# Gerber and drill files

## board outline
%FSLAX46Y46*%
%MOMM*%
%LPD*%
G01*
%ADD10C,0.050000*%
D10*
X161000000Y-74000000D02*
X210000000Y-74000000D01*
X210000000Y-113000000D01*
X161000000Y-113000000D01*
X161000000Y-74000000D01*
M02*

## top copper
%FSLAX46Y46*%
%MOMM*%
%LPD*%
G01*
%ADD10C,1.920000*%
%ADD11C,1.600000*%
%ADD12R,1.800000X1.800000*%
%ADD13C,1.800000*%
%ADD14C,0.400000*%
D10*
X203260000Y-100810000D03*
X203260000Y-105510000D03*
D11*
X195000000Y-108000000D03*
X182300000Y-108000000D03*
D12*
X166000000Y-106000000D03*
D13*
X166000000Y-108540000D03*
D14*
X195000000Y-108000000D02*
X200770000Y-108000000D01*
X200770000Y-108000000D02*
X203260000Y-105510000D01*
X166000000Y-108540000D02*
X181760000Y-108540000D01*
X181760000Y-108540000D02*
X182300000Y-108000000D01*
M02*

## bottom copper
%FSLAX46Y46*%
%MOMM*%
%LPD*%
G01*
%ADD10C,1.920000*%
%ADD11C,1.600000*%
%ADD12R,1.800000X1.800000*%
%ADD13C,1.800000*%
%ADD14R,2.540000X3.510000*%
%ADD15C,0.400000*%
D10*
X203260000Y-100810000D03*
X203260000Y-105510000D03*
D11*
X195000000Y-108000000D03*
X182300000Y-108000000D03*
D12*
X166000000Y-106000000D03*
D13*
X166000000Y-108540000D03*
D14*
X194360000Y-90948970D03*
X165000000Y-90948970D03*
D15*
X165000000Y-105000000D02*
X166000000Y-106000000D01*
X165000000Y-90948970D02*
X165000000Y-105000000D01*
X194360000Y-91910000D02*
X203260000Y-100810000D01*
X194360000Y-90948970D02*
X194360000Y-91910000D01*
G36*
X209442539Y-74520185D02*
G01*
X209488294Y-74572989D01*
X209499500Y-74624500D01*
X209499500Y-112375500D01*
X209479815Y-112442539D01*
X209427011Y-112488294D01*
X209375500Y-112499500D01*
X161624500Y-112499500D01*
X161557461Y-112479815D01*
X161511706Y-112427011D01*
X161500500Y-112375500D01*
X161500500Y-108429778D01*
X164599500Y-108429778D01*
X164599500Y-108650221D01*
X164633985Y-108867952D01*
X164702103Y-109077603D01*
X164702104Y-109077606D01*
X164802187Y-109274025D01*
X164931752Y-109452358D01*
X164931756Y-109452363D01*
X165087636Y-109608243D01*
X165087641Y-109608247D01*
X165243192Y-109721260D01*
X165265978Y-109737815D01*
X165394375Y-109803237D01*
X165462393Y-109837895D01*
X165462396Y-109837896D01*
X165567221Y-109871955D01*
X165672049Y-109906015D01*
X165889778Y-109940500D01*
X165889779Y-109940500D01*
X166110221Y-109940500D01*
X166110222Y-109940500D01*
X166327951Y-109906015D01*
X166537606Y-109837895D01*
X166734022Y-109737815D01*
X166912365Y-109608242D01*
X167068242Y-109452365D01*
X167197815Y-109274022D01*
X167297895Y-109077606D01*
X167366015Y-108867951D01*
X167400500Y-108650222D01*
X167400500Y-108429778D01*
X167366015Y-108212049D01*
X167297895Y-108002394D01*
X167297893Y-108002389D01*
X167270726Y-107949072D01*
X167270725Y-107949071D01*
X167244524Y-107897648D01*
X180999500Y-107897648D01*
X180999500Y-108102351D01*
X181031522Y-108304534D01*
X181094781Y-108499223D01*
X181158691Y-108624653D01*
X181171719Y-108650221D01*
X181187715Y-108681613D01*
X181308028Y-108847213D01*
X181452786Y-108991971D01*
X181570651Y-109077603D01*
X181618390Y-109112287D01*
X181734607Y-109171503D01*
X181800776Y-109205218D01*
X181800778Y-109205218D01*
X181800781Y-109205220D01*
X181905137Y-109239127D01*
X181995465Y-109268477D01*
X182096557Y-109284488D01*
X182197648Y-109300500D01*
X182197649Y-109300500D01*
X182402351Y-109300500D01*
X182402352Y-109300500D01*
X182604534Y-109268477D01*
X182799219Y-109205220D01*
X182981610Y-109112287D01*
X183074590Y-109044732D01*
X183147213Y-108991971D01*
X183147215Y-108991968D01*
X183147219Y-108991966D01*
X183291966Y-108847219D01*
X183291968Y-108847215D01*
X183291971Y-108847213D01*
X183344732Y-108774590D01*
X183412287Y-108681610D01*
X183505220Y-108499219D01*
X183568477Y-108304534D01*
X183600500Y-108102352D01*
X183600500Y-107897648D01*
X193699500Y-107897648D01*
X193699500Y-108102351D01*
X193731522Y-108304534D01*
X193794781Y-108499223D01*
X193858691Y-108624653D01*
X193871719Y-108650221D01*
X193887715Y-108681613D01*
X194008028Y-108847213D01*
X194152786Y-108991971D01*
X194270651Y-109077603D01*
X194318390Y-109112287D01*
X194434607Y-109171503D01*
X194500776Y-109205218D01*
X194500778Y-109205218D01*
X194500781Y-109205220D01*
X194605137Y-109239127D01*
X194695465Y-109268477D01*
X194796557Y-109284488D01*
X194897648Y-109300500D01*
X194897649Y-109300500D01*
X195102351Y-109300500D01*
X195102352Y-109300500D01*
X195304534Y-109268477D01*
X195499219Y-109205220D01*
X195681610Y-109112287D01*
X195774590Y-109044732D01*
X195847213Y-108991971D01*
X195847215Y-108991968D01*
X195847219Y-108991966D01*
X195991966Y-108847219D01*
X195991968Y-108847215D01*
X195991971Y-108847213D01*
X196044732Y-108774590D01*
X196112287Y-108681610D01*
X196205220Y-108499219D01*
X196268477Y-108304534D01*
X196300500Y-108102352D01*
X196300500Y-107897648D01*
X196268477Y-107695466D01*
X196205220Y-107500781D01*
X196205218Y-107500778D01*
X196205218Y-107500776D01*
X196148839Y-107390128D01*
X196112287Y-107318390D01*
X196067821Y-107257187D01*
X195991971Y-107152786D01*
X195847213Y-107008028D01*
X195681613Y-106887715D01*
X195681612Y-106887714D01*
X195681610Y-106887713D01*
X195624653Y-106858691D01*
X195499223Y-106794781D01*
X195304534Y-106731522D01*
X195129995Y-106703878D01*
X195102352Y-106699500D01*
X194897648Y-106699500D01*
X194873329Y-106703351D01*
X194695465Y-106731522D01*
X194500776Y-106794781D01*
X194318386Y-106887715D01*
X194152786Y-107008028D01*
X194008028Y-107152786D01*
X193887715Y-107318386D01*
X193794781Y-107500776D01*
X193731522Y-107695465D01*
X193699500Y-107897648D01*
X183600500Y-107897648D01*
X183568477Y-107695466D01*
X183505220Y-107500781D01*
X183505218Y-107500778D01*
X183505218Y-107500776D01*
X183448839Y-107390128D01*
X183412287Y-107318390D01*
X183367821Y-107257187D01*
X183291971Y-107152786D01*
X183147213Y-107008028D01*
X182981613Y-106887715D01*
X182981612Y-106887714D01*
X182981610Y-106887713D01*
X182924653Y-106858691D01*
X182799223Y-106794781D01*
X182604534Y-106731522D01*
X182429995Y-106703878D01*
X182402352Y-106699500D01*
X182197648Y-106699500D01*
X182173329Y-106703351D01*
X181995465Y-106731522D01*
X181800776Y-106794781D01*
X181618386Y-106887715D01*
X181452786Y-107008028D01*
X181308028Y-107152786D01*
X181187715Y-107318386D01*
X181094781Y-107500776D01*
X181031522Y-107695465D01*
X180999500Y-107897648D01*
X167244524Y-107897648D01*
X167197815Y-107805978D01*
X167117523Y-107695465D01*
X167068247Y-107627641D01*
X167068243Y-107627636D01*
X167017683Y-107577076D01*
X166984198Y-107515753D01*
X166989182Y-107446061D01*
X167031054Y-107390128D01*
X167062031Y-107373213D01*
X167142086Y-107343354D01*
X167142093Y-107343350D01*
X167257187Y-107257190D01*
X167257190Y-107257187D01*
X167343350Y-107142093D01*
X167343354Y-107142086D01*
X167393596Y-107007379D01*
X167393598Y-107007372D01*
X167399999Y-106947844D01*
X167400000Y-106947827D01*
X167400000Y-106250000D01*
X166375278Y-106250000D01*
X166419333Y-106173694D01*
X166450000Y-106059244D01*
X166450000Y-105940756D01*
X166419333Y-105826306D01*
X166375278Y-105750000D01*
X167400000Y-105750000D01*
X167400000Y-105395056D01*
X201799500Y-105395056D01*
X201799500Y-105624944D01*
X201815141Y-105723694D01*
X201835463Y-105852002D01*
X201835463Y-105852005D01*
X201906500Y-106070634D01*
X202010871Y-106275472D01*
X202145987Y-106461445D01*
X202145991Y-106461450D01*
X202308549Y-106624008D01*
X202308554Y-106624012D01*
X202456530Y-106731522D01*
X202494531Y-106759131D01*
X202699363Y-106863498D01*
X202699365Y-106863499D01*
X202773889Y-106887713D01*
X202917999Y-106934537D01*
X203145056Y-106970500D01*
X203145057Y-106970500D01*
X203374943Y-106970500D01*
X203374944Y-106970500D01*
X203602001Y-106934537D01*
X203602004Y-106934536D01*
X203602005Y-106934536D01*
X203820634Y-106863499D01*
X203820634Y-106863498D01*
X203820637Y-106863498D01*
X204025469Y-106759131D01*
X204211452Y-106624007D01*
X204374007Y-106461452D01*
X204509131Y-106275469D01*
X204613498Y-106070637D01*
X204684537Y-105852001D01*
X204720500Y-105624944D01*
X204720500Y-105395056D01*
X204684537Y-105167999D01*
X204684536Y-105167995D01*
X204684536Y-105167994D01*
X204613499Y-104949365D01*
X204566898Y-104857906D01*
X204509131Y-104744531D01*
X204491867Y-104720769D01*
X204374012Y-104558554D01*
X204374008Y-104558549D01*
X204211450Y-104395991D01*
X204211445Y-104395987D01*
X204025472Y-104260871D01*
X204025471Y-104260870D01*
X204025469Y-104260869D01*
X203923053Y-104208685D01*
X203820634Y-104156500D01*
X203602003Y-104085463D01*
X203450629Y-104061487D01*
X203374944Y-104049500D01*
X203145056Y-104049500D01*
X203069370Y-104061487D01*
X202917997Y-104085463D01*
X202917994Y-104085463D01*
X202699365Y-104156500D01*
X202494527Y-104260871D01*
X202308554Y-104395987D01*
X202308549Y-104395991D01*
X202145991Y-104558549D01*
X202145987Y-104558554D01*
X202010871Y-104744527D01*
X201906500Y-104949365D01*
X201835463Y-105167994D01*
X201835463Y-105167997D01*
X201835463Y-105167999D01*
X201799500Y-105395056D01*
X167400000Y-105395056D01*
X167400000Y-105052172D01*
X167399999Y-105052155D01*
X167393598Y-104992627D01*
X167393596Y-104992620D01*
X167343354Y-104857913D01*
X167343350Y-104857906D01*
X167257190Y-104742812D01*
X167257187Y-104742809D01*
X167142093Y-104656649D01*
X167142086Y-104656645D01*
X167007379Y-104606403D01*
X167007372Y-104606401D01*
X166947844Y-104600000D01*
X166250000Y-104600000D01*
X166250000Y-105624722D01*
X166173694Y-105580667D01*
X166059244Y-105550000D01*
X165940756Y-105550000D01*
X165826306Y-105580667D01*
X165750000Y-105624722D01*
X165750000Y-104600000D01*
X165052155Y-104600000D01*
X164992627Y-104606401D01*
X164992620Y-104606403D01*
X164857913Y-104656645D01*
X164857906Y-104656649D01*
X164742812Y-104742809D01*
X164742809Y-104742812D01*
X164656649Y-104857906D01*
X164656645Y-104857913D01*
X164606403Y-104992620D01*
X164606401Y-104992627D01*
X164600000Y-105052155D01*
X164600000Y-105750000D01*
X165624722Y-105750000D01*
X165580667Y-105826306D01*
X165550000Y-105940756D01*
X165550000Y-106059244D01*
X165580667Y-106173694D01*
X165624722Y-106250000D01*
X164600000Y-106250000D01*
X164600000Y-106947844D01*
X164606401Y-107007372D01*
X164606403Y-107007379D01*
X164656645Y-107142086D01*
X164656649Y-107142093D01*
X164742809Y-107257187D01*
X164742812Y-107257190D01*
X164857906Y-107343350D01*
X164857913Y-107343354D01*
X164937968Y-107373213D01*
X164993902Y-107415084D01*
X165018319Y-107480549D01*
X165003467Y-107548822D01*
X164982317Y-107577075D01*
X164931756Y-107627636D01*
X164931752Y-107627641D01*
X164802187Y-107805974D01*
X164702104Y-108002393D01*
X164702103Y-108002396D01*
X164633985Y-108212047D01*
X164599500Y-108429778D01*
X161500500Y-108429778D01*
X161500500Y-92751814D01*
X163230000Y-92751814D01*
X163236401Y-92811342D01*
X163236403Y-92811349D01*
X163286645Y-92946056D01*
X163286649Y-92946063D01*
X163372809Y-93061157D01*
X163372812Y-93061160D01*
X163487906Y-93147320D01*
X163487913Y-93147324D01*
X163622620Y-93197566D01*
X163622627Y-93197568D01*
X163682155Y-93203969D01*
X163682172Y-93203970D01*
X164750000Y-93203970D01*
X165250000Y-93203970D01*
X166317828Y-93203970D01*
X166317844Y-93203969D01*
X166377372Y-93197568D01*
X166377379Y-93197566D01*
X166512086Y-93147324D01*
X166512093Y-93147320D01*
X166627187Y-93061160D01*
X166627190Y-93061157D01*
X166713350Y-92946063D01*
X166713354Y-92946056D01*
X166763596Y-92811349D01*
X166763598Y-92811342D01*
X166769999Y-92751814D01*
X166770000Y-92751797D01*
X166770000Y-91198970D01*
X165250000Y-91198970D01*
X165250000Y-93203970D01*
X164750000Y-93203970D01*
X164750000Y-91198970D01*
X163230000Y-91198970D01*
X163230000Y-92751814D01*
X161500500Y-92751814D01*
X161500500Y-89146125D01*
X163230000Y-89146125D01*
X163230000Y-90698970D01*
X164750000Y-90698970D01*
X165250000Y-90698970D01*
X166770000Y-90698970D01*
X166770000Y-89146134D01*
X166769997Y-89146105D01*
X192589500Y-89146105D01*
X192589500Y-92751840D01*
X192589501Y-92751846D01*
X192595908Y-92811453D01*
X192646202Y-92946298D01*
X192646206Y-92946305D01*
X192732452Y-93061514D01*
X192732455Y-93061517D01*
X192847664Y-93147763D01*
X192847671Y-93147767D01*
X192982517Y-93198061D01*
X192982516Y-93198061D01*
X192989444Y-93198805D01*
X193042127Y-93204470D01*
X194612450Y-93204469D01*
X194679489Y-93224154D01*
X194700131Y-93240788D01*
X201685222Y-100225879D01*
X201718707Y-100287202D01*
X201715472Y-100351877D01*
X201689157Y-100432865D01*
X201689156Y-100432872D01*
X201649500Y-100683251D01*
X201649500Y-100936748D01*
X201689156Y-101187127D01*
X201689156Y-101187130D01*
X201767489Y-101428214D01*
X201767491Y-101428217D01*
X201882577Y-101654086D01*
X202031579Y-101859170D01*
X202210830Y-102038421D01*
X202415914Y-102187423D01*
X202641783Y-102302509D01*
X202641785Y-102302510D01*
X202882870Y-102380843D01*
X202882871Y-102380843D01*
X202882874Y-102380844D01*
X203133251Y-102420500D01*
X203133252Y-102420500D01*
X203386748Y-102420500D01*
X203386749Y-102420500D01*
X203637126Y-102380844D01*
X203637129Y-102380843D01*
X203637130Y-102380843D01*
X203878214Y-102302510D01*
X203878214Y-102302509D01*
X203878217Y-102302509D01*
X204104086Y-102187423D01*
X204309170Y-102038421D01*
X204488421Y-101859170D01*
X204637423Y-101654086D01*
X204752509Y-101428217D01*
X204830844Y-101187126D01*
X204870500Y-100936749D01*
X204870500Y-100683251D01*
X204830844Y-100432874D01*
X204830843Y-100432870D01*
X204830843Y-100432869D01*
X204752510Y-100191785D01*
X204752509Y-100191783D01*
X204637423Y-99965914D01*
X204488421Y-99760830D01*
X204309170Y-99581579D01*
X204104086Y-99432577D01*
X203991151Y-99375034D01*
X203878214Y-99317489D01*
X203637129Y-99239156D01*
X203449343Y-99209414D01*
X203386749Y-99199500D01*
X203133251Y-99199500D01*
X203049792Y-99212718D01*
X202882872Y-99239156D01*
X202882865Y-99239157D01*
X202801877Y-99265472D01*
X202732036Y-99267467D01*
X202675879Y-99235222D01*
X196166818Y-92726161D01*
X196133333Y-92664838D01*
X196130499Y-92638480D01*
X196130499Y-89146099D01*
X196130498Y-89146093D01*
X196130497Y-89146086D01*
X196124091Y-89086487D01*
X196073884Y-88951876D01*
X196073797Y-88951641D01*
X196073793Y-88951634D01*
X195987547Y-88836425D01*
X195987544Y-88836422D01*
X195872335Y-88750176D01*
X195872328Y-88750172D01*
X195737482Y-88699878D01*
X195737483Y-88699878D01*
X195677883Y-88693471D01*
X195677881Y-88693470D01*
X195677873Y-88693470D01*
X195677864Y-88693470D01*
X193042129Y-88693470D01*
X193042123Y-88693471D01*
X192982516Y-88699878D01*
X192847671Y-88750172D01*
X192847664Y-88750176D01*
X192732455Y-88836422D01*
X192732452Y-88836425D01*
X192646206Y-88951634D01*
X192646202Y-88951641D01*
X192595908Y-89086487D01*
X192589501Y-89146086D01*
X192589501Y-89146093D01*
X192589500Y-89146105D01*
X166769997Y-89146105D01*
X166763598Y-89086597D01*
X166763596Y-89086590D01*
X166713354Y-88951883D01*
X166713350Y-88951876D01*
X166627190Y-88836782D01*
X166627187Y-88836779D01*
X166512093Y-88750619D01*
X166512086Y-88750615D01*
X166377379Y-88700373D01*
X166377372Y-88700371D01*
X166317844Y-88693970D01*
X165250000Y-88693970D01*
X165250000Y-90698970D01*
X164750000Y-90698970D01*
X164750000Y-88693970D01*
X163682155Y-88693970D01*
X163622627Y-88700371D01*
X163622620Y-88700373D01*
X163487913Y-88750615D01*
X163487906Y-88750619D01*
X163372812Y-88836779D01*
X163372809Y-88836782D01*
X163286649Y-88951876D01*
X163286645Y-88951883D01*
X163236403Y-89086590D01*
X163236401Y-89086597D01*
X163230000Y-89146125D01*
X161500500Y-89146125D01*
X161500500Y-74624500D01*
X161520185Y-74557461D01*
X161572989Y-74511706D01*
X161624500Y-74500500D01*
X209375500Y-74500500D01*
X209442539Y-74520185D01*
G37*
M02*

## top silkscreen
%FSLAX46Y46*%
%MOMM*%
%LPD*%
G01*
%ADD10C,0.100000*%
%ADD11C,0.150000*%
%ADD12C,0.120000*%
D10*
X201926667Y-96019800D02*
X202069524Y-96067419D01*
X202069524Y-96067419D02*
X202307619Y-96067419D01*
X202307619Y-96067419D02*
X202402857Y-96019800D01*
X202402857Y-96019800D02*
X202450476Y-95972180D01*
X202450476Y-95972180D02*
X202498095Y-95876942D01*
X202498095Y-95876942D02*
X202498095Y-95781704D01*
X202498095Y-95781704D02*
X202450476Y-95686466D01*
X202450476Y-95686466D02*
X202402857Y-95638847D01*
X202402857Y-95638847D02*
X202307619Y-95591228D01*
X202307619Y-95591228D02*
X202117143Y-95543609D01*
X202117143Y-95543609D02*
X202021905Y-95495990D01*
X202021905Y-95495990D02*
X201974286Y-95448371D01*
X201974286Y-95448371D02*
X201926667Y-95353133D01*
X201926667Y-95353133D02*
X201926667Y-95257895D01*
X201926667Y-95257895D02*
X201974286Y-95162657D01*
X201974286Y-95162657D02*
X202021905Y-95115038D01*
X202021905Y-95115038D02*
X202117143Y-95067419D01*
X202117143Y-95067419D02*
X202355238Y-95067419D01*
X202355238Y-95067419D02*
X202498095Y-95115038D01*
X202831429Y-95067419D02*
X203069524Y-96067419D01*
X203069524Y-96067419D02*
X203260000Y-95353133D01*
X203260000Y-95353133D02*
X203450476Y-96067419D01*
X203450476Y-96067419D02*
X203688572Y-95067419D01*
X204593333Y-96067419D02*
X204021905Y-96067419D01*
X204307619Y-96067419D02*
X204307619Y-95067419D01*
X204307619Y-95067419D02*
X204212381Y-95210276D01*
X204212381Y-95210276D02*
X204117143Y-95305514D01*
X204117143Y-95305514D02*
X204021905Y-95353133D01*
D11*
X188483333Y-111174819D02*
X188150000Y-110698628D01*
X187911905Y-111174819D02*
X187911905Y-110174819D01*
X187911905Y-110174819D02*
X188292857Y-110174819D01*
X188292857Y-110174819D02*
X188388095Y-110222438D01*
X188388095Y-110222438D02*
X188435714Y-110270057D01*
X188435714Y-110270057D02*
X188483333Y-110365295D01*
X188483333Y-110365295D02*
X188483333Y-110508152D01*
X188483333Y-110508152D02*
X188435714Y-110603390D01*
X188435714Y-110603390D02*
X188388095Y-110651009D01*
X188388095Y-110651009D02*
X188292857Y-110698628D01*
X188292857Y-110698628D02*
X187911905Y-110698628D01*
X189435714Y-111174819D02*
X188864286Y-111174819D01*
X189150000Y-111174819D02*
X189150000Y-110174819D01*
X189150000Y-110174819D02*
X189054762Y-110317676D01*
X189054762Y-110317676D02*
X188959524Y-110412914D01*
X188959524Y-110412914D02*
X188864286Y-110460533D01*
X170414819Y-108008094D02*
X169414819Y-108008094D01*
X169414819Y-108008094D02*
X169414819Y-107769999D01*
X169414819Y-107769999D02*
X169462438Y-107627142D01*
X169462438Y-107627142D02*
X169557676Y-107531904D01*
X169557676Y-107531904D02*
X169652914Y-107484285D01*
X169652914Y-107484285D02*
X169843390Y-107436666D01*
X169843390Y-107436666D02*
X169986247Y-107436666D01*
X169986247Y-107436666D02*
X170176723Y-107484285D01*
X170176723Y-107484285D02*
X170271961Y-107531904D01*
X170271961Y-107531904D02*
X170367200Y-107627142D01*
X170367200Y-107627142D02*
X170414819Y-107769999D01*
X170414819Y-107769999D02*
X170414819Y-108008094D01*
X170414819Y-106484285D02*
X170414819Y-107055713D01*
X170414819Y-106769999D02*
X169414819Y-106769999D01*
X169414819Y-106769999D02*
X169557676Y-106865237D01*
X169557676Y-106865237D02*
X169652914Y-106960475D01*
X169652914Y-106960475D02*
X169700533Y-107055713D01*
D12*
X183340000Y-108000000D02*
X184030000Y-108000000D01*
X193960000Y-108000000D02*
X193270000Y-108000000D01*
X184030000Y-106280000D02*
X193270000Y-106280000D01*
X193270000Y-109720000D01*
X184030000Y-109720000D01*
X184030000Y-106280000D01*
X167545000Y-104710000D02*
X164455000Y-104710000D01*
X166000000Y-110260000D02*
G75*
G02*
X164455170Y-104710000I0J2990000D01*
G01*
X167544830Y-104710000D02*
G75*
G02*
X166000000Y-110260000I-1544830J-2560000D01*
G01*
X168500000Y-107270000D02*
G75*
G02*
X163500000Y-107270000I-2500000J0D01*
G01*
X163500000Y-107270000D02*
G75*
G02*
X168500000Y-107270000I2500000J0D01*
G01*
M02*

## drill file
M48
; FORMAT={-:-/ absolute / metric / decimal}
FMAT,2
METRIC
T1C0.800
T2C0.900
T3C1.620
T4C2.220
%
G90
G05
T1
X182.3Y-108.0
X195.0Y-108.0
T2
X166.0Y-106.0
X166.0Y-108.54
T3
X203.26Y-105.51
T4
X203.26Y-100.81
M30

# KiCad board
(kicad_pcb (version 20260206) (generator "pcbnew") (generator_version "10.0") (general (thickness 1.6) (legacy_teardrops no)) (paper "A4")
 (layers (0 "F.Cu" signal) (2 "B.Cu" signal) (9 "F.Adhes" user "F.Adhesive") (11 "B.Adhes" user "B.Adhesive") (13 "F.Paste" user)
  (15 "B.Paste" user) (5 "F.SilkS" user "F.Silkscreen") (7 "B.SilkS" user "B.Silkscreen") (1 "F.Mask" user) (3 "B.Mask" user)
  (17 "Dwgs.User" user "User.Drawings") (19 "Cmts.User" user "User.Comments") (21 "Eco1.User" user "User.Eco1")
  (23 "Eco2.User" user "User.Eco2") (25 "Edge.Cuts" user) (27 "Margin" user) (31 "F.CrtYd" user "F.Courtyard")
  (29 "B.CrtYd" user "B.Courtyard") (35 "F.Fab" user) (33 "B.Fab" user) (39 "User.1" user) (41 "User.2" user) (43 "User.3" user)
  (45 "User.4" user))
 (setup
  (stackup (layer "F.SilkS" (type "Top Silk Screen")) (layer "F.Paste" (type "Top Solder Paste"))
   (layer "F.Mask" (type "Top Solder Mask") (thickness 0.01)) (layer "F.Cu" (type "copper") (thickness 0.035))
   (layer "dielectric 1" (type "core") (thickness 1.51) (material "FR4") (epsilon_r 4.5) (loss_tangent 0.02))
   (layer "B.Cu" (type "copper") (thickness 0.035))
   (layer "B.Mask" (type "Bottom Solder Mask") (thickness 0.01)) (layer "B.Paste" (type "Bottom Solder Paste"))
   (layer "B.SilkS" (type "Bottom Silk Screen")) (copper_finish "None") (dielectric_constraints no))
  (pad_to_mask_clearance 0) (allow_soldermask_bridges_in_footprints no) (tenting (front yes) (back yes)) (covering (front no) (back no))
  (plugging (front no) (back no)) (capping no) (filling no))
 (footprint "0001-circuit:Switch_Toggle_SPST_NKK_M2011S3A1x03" (layer "F.Cu") (at 203.26 96.11)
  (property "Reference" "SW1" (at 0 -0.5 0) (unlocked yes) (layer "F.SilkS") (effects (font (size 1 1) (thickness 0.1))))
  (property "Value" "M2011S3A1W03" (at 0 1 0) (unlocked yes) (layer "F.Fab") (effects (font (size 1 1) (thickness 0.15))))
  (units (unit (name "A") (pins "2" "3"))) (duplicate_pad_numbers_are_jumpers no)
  (pad "2" thru_hole circle (at 0 4.7) (size 1.92 1.92) (drill 2.22) (layers "*.Cu" "*.Mask") (remove_unused_layers no) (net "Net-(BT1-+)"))
  (pad "3" thru_hole circle (at 0 9.4) (size 1.92 1.92) (drill 1.62) (layers "*.Cu" "*.Mask") (remove_unused_layers no) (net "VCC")))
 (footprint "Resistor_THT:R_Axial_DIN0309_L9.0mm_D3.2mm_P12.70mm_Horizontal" (layer "F.Cu") (at 195 108 180)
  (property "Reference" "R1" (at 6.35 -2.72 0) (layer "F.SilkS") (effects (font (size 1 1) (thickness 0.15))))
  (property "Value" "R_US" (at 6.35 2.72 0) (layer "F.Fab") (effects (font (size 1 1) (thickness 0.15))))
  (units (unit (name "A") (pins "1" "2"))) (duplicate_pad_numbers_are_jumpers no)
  (fp_line (start 11.66 0) (end 10.97 0) (stroke (width 0.12) (type solid)) (layer "F.SilkS"))
  (fp_line (start 1.04 0) (end 1.73 0) (stroke (width 0.12) (type solid)) (layer "F.SilkS"))
  (fp_rect (start 1.73 -1.72) (end 10.97 1.72) (stroke (width 0.12) (type solid)) (fill no) (layer "F.SilkS"))
  (pad "1" thru_hole circle (at 0 0 180) (size 1.6 1.6) (drill 0.8) (layers "*.Cu" "*.Mask") (remove_unused_layers no) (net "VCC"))
  (pad "2" thru_hole circle (at 12.7 0 180) (size 1.6 1.6) (drill 0.8) (layers "*.Cu" "*.Mask") (remove_unused_layers no) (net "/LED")))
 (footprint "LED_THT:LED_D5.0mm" (layer "F.Cu") (at 166 106 -90)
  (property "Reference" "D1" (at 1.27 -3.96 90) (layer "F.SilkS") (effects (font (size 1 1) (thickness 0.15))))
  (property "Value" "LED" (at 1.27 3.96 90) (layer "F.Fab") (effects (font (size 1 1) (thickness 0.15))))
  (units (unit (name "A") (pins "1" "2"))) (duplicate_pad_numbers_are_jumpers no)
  (fp_line (start -1.29 -1.545) (end -1.29 1.545) (stroke (width 0.12) (type solid)) (layer "F.SilkS"))
  (fp_arc (start 4.26 0) (mid 2.071779 2.880495) (end -1.29 1.54483) (stroke (width 0.12) (type solid)) (layer "F.SilkS"))
  (fp_arc (start -1.29 -1.54483) (mid 2.071779 -2.880495) (end 4.26 0) (stroke (width 0.12) (type solid)) (layer "F.SilkS"))
  (fp_circle (center 1.27 0) (end 3.77 0) (stroke (width 0.12) (type solid)) (fill no) (layer "F.SilkS"))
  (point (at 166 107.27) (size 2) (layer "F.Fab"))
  (pad "1" thru_hole rect (at 0 0 270) (size 1.8 1.8) (drill 0.9) (layers "*.Cu" "*.Mask") (remove_unused_layers no) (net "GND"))
  (pad "2" thru_hole circle (at 2.54 0 270) (size 1.8 1.8) (drill 0.9) (layers "*.Cu" "*.Mask") (remove_unused_layers no) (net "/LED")))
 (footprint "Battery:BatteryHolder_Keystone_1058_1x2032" (layer "B.Cu") (at 179.68 90.94897 180)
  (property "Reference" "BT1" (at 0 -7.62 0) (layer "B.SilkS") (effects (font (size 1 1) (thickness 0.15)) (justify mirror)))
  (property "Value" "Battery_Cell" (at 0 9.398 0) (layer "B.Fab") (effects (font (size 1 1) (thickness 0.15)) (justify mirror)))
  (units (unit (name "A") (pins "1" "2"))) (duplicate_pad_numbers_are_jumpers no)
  (pad "1" smd rect (at -14.68 0 180) (size 2.54 3.51) (layers "B.Cu" "B.Mask" "B.Paste") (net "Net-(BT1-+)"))
  (pad "2" smd rect (at 14.68 0 180) (size 2.54 3.51) (layers "B.Cu" "B.Mask" "B.Paste") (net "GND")))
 (gr_rect (start 161 74) (end 210 113) (stroke (width 0.05) (type default)) (fill no) (layer "Edge.Cuts"))
 (segment (start 195 108) (end 200.77 108) (width 0.4) (layer "F.Cu") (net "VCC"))
 (segment (start 200.77 108) (end 203.26 105.51) (width 0.4) (layer "F.Cu") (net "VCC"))
 (segment (start 166 108.54) (end 181.76 108.54) (width 0.4) (layer "F.Cu") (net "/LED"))
 (segment (start 181.76 108.54) (end 182.3 108) (width 0.4) (layer "F.Cu") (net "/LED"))
 (segment (start 165 105) (end 166 106) (width 0.4) (layer "B.Cu") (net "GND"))
 (segment (start 165 90.94897) (end 165 105) (width 0.4) (layer "B.Cu") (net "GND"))
 (segment (start 194.36 91.91) (end 203.26 100.81) (width 0.4) (layer "B.Cu") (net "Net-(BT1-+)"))
 (segment (start 194.36 90.94897) (end 194.36 91.91) (width 0.4) (layer "B.Cu") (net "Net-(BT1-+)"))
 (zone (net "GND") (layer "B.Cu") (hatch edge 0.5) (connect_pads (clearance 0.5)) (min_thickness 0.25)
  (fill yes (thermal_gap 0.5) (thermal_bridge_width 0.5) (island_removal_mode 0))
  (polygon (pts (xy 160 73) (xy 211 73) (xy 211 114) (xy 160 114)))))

